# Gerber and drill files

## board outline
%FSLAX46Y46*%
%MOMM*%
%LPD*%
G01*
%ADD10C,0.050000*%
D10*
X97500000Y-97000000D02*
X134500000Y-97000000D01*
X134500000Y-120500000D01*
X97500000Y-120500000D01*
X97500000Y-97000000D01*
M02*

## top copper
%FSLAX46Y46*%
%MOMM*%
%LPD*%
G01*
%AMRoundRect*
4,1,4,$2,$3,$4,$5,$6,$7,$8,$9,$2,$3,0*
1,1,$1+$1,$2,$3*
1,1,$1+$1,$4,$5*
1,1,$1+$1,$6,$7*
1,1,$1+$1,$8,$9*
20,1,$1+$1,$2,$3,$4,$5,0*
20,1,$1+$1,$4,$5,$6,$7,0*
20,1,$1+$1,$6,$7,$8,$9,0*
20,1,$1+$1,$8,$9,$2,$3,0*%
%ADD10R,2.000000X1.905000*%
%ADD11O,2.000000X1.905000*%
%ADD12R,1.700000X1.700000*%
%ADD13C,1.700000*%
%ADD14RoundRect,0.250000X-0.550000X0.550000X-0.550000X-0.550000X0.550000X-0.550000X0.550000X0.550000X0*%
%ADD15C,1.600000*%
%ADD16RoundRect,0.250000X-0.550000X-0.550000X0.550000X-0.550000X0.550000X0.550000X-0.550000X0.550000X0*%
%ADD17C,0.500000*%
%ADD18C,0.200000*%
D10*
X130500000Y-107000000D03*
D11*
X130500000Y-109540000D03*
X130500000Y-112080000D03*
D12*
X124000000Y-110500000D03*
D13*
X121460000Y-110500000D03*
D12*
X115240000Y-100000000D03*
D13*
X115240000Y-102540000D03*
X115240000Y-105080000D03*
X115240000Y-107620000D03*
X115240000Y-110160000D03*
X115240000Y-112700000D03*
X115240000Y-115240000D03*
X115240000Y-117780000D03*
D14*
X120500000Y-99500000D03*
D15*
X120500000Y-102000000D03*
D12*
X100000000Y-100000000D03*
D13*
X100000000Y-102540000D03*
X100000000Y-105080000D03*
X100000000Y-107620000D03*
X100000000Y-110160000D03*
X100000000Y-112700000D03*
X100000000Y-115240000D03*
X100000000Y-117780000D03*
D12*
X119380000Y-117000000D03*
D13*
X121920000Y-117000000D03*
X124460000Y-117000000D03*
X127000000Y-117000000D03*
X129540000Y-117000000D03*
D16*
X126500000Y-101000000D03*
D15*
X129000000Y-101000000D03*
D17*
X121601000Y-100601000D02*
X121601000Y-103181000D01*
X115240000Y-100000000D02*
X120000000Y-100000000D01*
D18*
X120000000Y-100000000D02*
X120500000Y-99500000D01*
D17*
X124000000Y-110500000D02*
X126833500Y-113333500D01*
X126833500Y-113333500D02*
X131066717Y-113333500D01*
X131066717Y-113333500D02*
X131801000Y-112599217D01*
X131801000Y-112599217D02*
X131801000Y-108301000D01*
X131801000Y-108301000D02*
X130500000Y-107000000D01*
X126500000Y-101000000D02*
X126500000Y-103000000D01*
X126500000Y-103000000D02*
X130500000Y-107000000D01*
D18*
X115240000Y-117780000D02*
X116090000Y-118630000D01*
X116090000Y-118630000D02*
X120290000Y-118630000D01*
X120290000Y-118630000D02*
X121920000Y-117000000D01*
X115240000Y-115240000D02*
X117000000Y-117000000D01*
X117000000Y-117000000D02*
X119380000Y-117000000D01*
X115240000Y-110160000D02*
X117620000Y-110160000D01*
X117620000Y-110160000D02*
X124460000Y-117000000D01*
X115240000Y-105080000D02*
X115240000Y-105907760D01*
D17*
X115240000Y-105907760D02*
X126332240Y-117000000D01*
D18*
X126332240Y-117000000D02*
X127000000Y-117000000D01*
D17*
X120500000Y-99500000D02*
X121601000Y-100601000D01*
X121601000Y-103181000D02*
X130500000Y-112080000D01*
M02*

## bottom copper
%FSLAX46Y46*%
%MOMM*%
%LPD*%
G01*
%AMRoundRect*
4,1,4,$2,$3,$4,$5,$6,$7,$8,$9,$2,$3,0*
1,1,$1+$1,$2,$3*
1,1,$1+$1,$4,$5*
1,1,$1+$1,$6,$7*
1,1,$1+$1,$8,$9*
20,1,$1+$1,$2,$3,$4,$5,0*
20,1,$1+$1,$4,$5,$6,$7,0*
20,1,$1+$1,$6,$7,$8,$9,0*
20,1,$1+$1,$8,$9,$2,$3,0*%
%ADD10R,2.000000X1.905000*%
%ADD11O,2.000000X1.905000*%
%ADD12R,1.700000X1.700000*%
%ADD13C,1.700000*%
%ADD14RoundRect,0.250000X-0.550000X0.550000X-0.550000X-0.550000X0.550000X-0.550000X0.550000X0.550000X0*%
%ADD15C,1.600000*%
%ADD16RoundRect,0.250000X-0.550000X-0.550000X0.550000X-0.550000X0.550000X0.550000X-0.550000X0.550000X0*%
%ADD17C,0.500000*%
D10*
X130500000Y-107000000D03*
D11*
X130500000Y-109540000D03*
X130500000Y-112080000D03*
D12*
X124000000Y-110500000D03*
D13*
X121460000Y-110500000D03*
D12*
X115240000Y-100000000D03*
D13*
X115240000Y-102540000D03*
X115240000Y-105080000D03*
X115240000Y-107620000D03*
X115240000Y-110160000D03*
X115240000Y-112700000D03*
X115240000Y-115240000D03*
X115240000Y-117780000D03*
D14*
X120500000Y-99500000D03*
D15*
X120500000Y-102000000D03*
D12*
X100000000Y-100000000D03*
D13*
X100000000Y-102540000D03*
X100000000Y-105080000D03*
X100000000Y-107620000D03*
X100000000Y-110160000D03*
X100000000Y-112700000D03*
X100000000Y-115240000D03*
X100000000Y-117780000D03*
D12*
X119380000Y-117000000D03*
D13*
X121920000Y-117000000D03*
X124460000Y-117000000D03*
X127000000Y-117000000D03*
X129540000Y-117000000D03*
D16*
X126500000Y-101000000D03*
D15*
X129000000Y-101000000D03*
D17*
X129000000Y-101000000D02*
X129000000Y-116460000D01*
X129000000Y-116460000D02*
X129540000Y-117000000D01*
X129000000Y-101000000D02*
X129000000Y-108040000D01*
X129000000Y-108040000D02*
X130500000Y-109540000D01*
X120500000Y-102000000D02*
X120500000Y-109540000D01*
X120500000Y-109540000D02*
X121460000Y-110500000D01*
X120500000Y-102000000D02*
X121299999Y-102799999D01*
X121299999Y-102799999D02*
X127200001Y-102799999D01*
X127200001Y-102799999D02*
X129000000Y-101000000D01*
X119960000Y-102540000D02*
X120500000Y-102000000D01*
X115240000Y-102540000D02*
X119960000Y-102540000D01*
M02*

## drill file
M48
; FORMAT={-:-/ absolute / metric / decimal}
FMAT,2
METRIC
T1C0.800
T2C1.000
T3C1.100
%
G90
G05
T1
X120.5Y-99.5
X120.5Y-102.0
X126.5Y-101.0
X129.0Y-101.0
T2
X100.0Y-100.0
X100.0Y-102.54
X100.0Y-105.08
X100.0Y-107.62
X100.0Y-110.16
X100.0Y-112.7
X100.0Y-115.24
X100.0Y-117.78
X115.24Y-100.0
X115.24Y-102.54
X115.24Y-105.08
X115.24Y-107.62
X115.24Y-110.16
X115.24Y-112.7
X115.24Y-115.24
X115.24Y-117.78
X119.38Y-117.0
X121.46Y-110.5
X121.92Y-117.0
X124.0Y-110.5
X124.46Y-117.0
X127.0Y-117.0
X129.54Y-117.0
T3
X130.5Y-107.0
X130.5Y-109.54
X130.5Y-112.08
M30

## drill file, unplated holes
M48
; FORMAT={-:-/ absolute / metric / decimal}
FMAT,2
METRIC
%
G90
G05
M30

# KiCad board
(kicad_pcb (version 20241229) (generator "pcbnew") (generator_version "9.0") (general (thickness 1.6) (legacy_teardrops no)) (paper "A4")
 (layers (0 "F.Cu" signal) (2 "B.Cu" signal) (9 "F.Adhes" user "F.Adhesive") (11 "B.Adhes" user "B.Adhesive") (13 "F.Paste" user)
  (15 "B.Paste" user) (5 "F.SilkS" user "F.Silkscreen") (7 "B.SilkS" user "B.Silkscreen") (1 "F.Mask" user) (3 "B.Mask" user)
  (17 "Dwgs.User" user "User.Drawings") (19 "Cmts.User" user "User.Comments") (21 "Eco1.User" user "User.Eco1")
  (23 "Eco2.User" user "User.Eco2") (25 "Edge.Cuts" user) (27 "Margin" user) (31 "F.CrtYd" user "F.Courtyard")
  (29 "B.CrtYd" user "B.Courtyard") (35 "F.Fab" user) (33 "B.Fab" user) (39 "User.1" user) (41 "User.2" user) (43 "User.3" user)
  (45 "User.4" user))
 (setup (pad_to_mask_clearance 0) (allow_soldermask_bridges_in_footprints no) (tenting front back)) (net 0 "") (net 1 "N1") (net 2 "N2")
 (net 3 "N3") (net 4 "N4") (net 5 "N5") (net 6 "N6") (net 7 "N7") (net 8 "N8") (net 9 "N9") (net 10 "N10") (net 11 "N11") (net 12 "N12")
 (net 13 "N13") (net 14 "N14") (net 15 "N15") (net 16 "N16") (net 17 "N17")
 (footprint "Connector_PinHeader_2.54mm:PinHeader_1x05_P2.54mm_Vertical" (layer "F.Cu") (at 119.38 117 90)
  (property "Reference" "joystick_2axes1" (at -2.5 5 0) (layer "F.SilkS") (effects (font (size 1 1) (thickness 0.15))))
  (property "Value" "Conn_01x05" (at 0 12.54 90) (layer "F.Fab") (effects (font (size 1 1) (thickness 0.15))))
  (pad "1" thru_hole rect (at 0 0 90) (size 1.7 1.7) (drill 1) (layers "*.Cu" "*.Mask") (remove_unused_layers no) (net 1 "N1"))
  (pad "2" thru_hole circle (at 0 2.54 90) (size 1.7 1.7) (drill 1) (layers "*.Cu" "*.Mask") (remove_unused_layers no) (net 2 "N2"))
  (pad "3" thru_hole circle (at 0 5.08 90) (size 1.7 1.7) (drill 1) (layers "*.Cu" "*.Mask") (remove_unused_layers no) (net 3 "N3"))
  (pad "4" thru_hole circle (at 0 7.62 90) (size 1.7 1.7) (drill 1) (layers "*.Cu" "*.Mask") (remove_unused_layers no) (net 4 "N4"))
  (pad "5" thru_hole circle (at 0 10.16 90) (size 1.7 1.7) (drill 1) (layers "*.Cu" "*.Mask") (remove_unused_layers no) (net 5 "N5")))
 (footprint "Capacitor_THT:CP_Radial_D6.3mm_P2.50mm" (layer "F.Cu") (at 126.5 101)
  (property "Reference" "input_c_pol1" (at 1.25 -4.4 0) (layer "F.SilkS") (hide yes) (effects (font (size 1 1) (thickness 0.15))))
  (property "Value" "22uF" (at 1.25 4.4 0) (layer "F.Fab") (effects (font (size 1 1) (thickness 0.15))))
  (pad "1" thru_hole roundrect (at 0 0) (size 1.6 1.6) (drill 0.8) (layers "*.Cu" "*.Mask") (remove_unused_layers no)
   (roundrect_rratio 0.15625) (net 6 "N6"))
  (pad "2" thru_hole circle (at 2.5 0) (size 1.6 1.6) (drill 0.8) (layers "*.Cu" "*.Mask") (remove_unused_layers no) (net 5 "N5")))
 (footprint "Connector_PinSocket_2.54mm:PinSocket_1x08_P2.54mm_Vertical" (layer "F.Cu") (at 100 100)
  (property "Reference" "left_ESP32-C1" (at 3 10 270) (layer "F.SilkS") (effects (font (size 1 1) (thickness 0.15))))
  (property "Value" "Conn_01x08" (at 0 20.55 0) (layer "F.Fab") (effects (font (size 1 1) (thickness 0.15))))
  (pad "1" thru_hole rect (at 0 0) (size 1.7 1.7) (drill 1) (layers "*.Cu" "*.Mask") (remove_unused_layers no) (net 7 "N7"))
  (pad "2" thru_hole circle (at 0 2.54) (size 1.7 1.7) (drill 1) (layers "*.Cu" "*.Mask") (remove_unused_layers no) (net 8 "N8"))
  (pad "3" thru_hole circle (at 0 5.08) (size 1.7 1.7) (drill 1) (layers "*.Cu" "*.Mask") (remove_unused_layers no) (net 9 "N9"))
  (pad "4" thru_hole circle (at 0 7.62) (size 1.7 1.7) (drill 1) (layers "*.Cu" "*.Mask") (remove_unused_layers no) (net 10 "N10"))
  (pad "5" thru_hole circle (at 0 10.16) (size 1.7 1.7) (drill 1) (layers "*.Cu" "*.Mask") (remove_unused_layers no) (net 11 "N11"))
  (pad "6" thru_hole circle (at 0 12.7) (size 1.7 1.7) (drill 1) (layers "*.Cu" "*.Mask") (remove_unused_layers no) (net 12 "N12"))
  (pad "7" thru_hole circle (at 0 15.24) (size 1.7 1.7) (drill 1) (layers "*.Cu" "*.Mask") (remove_unused_layers no) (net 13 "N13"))
  (pad "8" thru_hole circle (at 0 17.78) (size 1.7 1.7) (drill 1) (layers "*.Cu" "*.Mask") (remove_unused_layers no) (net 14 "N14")))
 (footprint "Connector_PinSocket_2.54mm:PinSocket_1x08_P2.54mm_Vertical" (layer "F.Cu") (at 115.24 100)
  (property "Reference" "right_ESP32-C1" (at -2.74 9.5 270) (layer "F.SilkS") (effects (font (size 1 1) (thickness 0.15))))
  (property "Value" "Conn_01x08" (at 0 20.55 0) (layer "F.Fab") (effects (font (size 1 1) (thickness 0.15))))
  (pad "1" thru_hole rect (at 0 0) (size 1.7 1.7) (drill 1) (layers "*.Cu" "*.Mask") (remove_unused_layers no) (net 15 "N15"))
  (pad "2" thru_hole circle (at 0 2.54) (size 1.7 1.7) (drill 1) (layers "*.Cu" "*.Mask") (remove_unused_layers no) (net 5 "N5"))
  (pad "3" thru_hole circle (at 0 5.08) (size 1.7 1.7) (drill 1) (layers "*.Cu" "*.Mask") (remove_unused_layers no) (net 4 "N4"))
  (pad "4" thru_hole circle (at 0 7.62) (size 1.7 1.7) (drill 1) (layers "*.Cu" "*.Mask") (remove_unused_layers no) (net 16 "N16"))
  (pad "5" thru_hole circle (at 0 10.16) (size 1.7 1.7) (drill 1) (layers "*.Cu" "*.Mask") (remove_unused_layers no) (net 3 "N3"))
  (pad "6" thru_hole circle (at 0 12.7) (size 1.7 1.7) (drill 1) (layers "*.Cu" "*.Mask") (remove_unused_layers no) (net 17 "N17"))
  (pad "7" thru_hole circle (at 0 15.24) (size 1.7 1.7) (drill 1) (layers "*.Cu" "*.Mask") (remove_unused_layers no) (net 1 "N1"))
  (pad "8" thru_hole circle (at 0 17.78) (size 1.7 1.7) (drill 1) (layers "*.Cu" "*.Mask") (remove_unused_layers no) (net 2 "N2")))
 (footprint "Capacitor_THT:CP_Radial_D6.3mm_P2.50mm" (layer "F.Cu") (at 120.5 99.5 -90)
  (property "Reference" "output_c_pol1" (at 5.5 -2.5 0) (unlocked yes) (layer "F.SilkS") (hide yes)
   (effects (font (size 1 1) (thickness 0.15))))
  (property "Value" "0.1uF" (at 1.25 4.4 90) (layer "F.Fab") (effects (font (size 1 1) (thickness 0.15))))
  (pad "1" thru_hole roundrect (at 0 0 270) (size 1.6 1.6) (drill 0.8) (layers "*.Cu" "*.Mask") (remove_unused_layers no)
   (roundrect_rratio 0.15625) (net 15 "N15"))
  (pad "2" thru_hole circle (at 2.5 0 270) (size 1.6 1.6) (drill 0.8) (layers "*.Cu" "*.Mask") (remove_unused_layers no) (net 5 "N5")))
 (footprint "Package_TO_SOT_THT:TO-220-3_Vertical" (layer "F.Cu") (at 130.5 107 -90)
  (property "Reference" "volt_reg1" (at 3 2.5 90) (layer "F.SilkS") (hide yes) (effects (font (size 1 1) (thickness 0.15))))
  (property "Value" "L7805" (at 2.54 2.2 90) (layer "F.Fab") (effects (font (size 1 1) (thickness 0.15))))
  (pad "1" thru_hole rect (at 0 0 270) (size 1.905 2) (drill 1.1) (layers "*.Cu" "*.Mask") (remove_unused_layers no) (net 6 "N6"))
  (pad "2" thru_hole oval (at 2.54 0 270) (size 1.905 2) (drill 1.1) (layers "*.Cu" "*.Mask") (remove_unused_layers no) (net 5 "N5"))
  (pad "3" thru_hole oval (at 5.08 0 270) (size 1.905 2) (drill 1.1) (layers "*.Cu" "*.Mask") (remove_unused_layers no) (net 15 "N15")))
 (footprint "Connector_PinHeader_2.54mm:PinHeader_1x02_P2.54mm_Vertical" (layer "F.Cu") (at 124 110.5 -90)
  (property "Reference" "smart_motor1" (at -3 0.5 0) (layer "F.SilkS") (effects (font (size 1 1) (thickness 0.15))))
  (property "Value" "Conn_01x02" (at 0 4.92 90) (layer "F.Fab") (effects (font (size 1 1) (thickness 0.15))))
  (pad "1" thru_hole rect (at 0 0 270) (size 1.7 1.7) (drill 1) (layers "*.Cu" "*.Mask") (remove_unused_layers no) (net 6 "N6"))
  (pad "2" thru_hole circle (at 0 2.54 270) (size 1.7 1.7) (drill 1) (layers "*.Cu" "*.Mask") (remove_unused_layers no) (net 5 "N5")))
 (gr_rect (start 97.5 97) (end 134.5 120.5) (stroke (width 0.05) (type default)) (fill no) (layer "Edge.Cuts"))
 (segment (start 126.5 103) (end 130.5 107) (width 0.5) (layer "F.Cu") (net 6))
 (segment (start 126.8335 113.3335) (end 131.066717 113.3335) (width 0.5) (layer "F.Cu") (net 6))
 (segment (start 124 110.5) (end 126.8335 113.3335) (width 0.5) (layer "F.Cu") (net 6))
 (segment (start 131.066717 113.3335) (end 131.801 112.599217) (width 0.5) (layer "F.Cu") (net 6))
 (segment (start 131.801 112.599217) (end 131.801 108.301) (width 0.5) (layer "F.Cu") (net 6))
 (segment (start 131.801 108.301) (end 130.5 107) (width 0.5) (layer "F.Cu") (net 6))
 (segment (start 126.5 101) (end 126.5 103) (width 0.5) (layer "F.Cu") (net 6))
 (segment (start 127.200001 102.799999) (end 129 101) (width 0.5) (layer "B.Cu") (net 5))
 (segment (start 129 108.04) (end 130.5 109.54) (width 0.5) (layer "B.Cu") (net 5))
 (segment (start 129 101) (end 129 116.46) (width 0.5) (layer "B.Cu") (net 5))
 (segment (start 129 101) (end 129 108.04) (width 0.5) (layer "B.Cu") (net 5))
 (segment (start 120.5 102) (end 121.299999 102.799999) (width 0.5) (layer "B.Cu") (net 5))
 (segment (start 121.299999 102.799999) (end 127.200001 102.799999) (width 0.5) (layer "B.Cu") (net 5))
 (segment (start 120.5 109.54) (end 121.46 110.5) (width 0.5) (layer "B.Cu") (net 5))
 (segment (start 129 116.46) (end 129.54 117) (width 0.5) (layer "B.Cu") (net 5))
 (segment (start 119.96 102.54) (end 120.5 102) (width 0.5) (layer "B.Cu") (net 5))
 (segment (start 115.24 102.54) (end 119.96 102.54) (width 0.5) (layer "B.Cu") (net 5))
 (segment (start 120.5 102) (end 120.5 109.54) (width 0.5) (layer "B.Cu") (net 5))
 (segment (start 115.24 105.90776) (end 126.33224 117) (width 0.5) (layer "F.Cu") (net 4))
 (segment (start 115.24 105.08) (end 115.24 105.90776) (width 0.2) (layer "F.Cu") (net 4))
 (segment (start 126.33224 117) (end 127 117) (width 0.2) (layer "F.Cu") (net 4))
 (segment (start 120.29 118.63) (end 121.92 117) (width 0.2) (layer "F.Cu") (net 2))
 (segment (start 116.09 118.63) (end 120.29 118.63) (width 0.2) (layer "F.Cu") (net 2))
 (segment (start 115.24 117.78) (end 116.09 118.63) (width 0.2) (layer "F.Cu") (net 2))
 (segment (start 117 117) (end 119.38 117) (width 0.2) (layer "F.Cu") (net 1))
 (segment (start 115.24 115.24) (end 117 117) (width 0.2) (layer "F.Cu") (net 1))
 (segment (start 115.24 110.16) (end 117.62 110.16) (width 0.2) (layer "F.Cu") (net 3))
 (segment (start 117.62 110.16) (end 124.46 117) (width 0.2) (layer "F.Cu") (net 3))
 (segment (start 115.24 100) (end 120 100) (width 0.5) (layer "F.Cu") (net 15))
 (segment (start 121.601 100.601) (end 121.601 103.181) (width 0.5) (layer "F.Cu") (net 15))
 (segment (start 120 100) (end 120.5 99.5) (width 0.2) (layer "F.Cu") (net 15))
 (segment (start 120.5 99.5) (end 121.601 100.601) (width 0.5) (layer "F.Cu") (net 15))
 (segment (start 121.601 103.181) (end 130.5 112.08) (width 0.5) (layer "F.Cu") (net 15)))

